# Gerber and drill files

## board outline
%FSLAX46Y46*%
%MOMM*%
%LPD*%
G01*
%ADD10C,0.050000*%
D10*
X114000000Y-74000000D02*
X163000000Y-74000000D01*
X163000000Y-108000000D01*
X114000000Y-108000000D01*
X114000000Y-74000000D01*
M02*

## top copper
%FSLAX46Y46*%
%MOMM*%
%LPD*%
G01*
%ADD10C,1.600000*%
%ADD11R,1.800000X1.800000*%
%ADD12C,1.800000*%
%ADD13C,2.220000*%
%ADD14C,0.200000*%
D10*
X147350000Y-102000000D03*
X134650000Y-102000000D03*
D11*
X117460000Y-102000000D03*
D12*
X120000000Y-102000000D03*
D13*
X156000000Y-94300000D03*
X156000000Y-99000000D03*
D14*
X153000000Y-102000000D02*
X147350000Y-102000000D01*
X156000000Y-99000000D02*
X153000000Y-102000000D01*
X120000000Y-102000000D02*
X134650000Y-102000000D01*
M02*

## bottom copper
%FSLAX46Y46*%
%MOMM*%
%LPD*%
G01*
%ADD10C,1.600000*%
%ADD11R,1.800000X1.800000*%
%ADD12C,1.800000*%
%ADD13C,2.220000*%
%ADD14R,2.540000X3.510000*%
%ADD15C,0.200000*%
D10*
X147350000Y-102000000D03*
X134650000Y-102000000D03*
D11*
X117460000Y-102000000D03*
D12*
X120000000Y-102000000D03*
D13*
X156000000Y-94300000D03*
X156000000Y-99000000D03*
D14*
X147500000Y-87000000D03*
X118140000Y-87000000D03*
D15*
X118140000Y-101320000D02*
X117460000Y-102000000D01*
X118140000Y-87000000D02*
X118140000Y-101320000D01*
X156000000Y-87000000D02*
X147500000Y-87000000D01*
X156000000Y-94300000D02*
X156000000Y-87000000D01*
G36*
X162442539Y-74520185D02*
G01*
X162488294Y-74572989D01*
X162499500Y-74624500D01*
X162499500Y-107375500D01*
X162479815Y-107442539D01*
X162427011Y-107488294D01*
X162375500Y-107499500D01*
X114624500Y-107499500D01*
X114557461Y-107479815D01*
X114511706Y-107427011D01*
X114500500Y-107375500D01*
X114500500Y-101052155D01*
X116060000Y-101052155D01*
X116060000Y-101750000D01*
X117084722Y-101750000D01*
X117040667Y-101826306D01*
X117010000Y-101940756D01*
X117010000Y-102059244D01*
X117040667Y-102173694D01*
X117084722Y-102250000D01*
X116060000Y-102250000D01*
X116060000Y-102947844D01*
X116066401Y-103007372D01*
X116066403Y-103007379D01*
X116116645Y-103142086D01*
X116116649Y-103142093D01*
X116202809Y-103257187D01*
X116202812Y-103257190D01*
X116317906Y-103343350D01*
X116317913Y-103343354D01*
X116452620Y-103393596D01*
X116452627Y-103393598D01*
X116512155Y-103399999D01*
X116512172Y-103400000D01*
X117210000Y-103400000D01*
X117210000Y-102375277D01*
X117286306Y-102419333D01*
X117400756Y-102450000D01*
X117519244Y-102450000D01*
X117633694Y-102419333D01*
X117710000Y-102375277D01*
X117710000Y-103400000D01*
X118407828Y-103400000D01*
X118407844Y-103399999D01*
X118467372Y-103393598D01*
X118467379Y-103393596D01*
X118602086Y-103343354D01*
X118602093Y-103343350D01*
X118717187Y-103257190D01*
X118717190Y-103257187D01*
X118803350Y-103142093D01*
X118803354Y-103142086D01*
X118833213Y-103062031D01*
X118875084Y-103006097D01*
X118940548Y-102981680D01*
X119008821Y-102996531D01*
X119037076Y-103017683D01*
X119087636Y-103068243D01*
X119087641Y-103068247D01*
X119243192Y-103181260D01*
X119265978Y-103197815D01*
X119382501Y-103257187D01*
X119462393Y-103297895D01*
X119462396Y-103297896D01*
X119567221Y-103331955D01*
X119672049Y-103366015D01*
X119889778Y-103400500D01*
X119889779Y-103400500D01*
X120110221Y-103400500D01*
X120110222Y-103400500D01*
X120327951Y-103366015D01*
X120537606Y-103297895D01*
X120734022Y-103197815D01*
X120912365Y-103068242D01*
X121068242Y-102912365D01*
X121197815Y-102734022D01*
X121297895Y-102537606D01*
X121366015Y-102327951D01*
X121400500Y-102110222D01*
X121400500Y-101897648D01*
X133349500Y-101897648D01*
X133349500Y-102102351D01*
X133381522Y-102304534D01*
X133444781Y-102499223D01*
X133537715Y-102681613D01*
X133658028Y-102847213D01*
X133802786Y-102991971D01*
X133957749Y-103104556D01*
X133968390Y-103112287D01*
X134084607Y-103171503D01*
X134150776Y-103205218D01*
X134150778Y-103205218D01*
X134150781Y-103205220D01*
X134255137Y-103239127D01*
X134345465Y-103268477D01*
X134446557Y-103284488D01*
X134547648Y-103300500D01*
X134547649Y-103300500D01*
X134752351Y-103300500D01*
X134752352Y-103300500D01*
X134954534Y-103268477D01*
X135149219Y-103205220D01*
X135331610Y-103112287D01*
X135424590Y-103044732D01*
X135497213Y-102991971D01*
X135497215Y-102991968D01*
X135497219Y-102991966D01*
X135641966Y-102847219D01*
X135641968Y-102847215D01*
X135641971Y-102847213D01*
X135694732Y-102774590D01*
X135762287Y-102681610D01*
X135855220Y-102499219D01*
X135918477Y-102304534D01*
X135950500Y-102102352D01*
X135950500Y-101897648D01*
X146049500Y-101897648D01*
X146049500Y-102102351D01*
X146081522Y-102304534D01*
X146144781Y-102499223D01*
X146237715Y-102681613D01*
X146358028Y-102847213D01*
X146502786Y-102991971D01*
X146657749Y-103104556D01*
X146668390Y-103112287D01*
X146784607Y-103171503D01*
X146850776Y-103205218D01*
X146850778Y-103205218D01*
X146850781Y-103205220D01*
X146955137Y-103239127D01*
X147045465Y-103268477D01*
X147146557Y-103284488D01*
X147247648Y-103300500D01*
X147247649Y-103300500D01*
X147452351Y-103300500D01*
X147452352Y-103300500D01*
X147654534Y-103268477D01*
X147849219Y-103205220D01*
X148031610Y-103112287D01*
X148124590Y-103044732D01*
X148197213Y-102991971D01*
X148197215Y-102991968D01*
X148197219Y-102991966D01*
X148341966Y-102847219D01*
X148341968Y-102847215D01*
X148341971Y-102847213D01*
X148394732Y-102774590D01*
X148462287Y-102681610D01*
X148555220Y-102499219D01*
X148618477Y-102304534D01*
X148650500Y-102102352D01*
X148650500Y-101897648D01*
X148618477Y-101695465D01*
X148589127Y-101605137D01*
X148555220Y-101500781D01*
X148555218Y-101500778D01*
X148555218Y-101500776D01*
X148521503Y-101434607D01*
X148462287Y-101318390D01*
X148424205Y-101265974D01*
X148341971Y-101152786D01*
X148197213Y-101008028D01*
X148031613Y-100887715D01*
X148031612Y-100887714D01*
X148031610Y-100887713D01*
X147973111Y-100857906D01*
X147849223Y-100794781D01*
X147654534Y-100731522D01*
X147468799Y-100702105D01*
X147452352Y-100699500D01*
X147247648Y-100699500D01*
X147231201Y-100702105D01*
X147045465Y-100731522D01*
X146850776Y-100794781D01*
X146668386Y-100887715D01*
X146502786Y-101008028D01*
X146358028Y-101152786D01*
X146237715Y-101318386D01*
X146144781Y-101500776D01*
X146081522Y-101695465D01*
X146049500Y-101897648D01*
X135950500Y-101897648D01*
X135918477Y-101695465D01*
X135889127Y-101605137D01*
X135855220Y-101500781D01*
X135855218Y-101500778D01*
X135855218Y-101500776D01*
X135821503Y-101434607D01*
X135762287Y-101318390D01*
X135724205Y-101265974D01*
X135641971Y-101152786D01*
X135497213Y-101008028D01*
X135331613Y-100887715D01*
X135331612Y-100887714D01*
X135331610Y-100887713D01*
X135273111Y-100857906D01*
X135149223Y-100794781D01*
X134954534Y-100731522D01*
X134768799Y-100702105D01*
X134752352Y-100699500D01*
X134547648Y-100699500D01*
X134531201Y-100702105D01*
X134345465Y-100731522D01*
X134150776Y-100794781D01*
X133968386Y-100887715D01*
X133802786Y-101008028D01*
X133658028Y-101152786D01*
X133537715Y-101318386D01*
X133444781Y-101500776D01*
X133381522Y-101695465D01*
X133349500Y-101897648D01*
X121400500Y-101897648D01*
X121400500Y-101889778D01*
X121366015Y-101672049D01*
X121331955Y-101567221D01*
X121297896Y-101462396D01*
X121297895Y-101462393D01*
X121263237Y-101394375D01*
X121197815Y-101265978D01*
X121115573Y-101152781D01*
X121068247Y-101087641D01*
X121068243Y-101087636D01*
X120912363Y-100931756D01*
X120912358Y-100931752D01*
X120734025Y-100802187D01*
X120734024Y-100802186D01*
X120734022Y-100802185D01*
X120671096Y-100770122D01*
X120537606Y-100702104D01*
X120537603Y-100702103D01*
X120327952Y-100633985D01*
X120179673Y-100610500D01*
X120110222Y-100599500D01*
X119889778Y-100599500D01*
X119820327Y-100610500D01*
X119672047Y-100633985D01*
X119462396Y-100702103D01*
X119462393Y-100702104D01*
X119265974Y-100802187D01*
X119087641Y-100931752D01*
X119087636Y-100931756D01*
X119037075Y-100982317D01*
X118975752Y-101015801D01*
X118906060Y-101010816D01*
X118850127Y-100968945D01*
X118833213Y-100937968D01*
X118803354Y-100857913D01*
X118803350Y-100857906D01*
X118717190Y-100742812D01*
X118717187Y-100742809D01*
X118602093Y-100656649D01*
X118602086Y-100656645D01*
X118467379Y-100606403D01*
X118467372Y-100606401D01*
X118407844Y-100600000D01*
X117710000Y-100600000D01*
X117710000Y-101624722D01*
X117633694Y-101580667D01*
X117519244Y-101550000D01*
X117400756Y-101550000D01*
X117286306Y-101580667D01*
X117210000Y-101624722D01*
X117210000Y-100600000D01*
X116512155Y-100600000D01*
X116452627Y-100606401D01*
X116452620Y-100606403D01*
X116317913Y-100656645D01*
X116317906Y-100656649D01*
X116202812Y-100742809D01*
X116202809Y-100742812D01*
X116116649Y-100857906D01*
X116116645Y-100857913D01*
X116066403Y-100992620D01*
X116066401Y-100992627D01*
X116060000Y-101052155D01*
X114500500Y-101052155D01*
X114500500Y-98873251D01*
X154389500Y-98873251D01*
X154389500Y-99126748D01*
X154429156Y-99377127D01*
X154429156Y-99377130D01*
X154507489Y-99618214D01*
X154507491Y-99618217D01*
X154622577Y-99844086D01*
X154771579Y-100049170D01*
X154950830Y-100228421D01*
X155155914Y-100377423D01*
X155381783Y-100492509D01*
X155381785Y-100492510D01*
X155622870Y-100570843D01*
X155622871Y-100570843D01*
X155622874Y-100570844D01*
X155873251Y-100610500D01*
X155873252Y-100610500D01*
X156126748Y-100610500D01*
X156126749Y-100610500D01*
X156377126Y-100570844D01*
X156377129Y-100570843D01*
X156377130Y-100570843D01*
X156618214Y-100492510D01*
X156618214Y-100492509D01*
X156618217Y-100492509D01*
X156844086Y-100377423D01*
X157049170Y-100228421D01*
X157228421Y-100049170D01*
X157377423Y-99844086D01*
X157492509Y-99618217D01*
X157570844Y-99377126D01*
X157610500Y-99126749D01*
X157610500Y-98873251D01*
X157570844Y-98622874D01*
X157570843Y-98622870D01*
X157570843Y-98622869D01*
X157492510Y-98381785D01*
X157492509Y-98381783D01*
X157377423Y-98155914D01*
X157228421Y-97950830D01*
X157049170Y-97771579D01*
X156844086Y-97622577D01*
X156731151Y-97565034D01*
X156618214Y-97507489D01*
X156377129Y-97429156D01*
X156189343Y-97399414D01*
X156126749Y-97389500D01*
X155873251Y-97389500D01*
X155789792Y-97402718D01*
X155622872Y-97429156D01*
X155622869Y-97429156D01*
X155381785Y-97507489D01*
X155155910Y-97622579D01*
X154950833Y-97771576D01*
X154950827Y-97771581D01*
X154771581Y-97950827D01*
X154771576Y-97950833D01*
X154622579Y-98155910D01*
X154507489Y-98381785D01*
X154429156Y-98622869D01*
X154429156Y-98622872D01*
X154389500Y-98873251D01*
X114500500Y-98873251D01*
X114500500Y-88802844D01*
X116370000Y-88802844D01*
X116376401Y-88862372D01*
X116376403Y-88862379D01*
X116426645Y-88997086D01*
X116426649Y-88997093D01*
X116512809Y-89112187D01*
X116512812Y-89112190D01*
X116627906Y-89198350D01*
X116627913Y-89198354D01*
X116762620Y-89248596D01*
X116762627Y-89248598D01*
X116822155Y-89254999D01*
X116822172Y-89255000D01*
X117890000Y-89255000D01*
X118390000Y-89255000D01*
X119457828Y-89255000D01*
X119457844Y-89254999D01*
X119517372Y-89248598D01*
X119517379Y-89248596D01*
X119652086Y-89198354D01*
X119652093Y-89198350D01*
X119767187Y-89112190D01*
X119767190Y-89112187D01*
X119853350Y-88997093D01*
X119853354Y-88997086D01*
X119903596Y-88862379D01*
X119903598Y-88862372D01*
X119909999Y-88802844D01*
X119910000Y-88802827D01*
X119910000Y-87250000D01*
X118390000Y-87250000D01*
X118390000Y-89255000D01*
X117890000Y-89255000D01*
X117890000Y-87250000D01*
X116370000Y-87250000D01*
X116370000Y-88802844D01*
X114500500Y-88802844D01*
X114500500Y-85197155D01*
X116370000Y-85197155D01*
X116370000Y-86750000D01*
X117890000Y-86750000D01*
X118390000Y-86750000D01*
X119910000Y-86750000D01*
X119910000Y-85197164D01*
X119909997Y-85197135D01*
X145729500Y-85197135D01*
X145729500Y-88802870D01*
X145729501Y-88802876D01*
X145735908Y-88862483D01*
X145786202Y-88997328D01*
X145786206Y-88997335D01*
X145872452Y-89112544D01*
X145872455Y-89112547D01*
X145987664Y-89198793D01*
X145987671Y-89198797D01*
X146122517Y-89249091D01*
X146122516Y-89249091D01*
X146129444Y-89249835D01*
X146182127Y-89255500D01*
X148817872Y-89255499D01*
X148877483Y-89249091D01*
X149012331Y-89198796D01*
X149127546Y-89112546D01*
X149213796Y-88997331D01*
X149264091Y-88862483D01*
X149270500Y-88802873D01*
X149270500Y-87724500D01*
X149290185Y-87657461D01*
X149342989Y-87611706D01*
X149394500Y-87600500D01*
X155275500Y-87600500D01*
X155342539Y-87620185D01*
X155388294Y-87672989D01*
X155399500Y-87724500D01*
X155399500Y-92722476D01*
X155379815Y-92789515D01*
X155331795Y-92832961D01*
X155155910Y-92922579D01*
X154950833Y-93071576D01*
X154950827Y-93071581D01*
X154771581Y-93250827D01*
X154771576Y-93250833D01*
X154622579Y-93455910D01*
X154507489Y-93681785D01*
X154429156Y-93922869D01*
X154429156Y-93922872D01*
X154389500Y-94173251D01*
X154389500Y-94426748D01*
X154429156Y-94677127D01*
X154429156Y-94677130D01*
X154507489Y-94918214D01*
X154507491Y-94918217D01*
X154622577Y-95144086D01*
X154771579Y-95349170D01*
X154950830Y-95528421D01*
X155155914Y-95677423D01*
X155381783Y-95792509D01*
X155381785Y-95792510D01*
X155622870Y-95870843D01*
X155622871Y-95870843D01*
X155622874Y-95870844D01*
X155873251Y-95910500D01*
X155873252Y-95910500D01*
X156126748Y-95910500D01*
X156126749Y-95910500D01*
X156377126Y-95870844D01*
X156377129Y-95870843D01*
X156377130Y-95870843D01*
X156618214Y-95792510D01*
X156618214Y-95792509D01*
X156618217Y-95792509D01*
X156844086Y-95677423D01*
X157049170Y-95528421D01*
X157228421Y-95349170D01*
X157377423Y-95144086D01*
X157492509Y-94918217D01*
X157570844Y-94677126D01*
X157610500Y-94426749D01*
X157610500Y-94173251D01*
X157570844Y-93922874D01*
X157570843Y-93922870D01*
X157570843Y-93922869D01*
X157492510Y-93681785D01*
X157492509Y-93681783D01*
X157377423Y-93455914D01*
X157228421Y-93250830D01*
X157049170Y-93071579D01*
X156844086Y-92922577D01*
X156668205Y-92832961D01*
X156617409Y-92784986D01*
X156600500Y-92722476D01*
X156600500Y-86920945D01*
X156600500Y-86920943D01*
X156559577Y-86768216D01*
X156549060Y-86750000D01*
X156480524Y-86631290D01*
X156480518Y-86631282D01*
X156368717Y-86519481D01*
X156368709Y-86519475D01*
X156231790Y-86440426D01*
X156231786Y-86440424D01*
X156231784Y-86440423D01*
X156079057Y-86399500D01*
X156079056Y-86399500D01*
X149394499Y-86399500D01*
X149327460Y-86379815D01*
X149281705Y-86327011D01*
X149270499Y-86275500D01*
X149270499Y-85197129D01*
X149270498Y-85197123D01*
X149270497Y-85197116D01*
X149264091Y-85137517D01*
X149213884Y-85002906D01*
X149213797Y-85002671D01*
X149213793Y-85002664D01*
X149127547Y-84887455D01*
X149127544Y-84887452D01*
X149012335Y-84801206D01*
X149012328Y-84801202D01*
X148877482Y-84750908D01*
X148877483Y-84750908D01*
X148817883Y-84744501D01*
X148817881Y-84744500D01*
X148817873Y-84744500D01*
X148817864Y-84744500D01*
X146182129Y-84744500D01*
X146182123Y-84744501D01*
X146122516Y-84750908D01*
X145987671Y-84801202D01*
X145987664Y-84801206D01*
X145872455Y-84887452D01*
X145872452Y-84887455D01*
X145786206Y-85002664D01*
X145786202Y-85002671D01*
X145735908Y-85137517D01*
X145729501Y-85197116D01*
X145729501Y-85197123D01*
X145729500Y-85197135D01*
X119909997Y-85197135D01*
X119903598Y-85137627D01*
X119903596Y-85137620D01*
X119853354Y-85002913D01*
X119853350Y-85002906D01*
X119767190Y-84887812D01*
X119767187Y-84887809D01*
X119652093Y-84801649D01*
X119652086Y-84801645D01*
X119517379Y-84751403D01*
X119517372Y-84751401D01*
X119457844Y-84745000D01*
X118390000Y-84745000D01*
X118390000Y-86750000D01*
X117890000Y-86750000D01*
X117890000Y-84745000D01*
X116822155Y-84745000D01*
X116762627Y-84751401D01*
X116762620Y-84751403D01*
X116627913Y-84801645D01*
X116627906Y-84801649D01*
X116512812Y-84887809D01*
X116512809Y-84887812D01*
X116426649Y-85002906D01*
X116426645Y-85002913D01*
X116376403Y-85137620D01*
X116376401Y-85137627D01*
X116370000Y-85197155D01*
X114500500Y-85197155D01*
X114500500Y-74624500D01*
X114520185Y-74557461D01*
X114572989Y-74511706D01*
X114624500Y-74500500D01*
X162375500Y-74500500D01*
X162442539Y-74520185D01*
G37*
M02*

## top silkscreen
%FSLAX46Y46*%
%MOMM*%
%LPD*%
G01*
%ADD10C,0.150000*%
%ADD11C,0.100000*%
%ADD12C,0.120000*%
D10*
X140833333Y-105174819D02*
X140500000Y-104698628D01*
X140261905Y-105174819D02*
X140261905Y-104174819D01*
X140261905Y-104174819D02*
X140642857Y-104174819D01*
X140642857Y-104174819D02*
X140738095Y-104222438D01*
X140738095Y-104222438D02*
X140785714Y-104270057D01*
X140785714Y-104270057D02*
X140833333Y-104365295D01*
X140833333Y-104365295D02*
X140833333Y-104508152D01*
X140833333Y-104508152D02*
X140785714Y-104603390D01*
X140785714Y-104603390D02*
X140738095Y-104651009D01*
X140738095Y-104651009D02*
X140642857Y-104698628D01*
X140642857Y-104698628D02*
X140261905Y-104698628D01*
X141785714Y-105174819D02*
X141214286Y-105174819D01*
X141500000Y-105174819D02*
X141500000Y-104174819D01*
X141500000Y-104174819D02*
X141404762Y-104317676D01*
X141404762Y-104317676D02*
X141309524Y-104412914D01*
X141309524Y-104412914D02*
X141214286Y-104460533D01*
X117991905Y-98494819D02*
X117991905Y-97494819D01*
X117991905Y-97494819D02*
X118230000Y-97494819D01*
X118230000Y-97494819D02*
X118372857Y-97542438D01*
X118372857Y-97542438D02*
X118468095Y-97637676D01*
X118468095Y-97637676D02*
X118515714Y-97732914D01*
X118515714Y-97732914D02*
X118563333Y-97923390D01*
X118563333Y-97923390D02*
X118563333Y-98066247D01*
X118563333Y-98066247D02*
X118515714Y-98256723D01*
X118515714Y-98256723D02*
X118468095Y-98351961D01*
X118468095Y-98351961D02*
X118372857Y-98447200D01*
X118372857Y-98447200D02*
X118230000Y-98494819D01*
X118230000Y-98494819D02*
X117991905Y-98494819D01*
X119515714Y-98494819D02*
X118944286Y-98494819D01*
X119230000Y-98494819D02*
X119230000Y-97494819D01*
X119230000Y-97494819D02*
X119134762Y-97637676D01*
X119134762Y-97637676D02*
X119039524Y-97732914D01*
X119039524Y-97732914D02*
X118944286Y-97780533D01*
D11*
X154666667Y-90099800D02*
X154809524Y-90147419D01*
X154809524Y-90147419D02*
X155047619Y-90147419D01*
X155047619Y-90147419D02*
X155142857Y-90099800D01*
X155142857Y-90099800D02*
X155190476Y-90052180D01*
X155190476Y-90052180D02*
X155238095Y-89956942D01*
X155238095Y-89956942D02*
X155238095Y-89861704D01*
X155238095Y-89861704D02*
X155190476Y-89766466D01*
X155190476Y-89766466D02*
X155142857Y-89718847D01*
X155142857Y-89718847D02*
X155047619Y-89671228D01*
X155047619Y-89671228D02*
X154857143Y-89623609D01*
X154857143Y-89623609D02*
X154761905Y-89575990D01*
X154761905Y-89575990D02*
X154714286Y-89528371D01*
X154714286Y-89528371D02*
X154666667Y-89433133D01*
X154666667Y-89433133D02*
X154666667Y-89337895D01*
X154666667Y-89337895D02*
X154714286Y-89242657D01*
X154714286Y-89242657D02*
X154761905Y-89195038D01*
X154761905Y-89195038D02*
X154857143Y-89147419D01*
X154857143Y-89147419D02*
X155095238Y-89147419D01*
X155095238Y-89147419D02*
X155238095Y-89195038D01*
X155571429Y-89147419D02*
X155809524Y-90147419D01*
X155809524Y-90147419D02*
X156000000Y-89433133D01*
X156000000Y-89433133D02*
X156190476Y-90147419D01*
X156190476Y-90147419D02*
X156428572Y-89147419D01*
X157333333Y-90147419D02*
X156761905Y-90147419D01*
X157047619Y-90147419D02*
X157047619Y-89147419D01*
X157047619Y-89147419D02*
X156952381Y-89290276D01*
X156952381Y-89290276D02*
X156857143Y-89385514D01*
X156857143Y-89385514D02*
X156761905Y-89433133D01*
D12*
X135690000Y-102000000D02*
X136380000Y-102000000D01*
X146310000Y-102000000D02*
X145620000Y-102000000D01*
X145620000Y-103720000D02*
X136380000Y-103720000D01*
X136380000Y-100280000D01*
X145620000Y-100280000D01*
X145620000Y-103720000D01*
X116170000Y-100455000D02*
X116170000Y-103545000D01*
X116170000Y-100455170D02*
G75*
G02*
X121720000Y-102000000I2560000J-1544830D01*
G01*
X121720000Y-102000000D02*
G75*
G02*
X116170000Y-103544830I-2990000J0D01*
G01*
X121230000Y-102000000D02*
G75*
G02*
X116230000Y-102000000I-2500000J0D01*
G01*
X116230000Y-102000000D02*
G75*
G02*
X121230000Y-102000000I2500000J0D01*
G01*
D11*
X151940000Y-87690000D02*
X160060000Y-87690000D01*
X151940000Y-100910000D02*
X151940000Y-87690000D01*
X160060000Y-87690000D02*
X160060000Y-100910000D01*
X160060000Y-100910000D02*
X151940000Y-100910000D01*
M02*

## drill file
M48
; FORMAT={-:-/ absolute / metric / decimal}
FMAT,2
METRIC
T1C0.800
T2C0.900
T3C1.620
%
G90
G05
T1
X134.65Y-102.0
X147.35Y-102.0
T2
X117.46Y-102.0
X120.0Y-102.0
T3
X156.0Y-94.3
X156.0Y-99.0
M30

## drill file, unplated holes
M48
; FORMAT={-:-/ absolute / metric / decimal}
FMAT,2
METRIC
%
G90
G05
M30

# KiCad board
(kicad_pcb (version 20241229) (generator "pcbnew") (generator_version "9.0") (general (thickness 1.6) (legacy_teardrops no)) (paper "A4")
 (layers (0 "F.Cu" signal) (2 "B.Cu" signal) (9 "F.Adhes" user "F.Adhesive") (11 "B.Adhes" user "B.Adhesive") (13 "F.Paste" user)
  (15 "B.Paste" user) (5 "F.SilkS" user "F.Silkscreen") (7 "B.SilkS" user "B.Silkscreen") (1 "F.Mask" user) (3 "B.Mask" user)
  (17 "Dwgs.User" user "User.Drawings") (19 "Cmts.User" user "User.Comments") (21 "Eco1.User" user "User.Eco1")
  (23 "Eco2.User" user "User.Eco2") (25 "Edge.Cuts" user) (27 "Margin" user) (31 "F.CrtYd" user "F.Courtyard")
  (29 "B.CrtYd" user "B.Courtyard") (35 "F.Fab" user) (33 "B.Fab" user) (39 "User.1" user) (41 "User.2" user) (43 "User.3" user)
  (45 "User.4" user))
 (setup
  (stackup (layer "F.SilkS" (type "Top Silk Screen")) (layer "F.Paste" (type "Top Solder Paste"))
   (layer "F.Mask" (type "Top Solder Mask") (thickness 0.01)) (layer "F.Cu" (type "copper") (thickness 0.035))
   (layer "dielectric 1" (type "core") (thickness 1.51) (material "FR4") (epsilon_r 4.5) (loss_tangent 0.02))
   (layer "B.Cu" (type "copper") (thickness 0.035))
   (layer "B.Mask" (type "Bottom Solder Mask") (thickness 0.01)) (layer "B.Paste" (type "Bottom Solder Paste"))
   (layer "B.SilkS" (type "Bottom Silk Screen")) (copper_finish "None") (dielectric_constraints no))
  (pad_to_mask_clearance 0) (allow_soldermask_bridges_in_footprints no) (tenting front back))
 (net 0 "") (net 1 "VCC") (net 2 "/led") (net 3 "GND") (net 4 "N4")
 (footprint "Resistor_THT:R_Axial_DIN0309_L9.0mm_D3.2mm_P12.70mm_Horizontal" (layer "F.Cu") (at 147.35 102 180)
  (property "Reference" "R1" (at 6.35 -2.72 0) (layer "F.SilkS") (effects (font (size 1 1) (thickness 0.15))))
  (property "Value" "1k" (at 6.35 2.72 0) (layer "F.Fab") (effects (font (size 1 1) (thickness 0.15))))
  (fp_line (start 11.66 0) (end 10.97 0) (stroke (width 0.12) (type solid)) (layer "F.SilkS"))
  (fp_line (start 1.04 0) (end 1.73 0) (stroke (width 0.12) (type solid)) (layer "F.SilkS"))
  (fp_rect (start 1.73 -1.72) (end 10.97 1.72) (stroke (width 0.12) (type solid)) (fill no) (layer "F.SilkS"))
  (pad "1" thru_hole circle (at 0 0 180) (size 1.6 1.6) (drill 0.8) (layers "*.Cu" "*.Mask") (remove_unused_layers no) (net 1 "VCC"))
  (pad "2" thru_hole circle (at 12.7 0 180) (size 1.6 1.6) (drill 0.8) (layers "*.Cu" "*.Mask") (remove_unused_layers no) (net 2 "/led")))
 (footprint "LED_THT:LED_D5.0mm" (layer "F.Cu") (at 117.46 102)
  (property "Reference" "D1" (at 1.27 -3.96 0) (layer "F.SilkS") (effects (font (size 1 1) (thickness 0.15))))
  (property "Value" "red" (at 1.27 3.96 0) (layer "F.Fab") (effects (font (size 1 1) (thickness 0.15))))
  (fp_line (start -1.29 -1.545) (end -1.29 1.545) (stroke (width 0.12) (type solid)) (layer "F.SilkS"))
  (fp_arc (start -1.29 -1.54483) (mid 2.071779 -2.880495) (end 4.26 0) (stroke (width 0.12) (type solid)) (layer "F.SilkS"))
  (fp_arc (start 4.26 0) (mid 2.071779 2.880495) (end -1.29 1.54483) (stroke (width 0.12) (type solid)) (layer "F.SilkS"))
  (fp_circle (center 1.27 0) (end 3.77 0) (stroke (width 0.12) (type solid)) (fill no) (layer "F.SilkS"))
  (pad "1" thru_hole rect (at 0 0) (size 1.8 1.8) (drill 0.9) (layers "*.Cu" "*.Mask") (remove_unused_layers no) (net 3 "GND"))
  (pad "2" thru_hole circle (at 2.54 0) (size 1.8 1.8) (drill 0.9) (layers "*.Cu" "*.Mask") (remove_unused_layers no) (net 2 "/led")))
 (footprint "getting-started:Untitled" (layer "F.Cu") (at 156 89.6)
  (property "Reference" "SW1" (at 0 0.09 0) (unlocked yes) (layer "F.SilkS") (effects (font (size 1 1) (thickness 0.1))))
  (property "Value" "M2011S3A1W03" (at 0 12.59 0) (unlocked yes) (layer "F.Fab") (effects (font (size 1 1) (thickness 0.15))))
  (fp_line (start -4.06 -1.91) (end 4.06 -1.91) (stroke (width 0.1) (type default)) (layer "F.SilkS"))
  (fp_line (start -4.06 11.31) (end -4.06 -1.91) (stroke (width 0.1) (type default)) (layer "F.SilkS"))
  (fp_line (start 4.06 -1.91) (end 4.06 11.31) (stroke (width 0.1) (type default)) (layer "F.SilkS"))
  (fp_line (start 4.06 11.31) (end -4.06 11.31) (stroke (width 0.1) (type default)) (layer "F.SilkS"))
  (pad "2" thru_hole circle (at 0 4.7) (size 2.22 2.22) (drill 1.62) (layers "*.Cu" "*.Mask") (remove_unused_layers no) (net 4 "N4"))
  (pad "3" thru_hole circle (at 0 9.4) (size 2.22 2.22) (drill 1.62) (layers "*.Cu" "*.Mask") (remove_unused_layers no) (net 1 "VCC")))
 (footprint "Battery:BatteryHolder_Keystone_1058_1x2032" (layer "B.Cu") (at 132.82 87 180)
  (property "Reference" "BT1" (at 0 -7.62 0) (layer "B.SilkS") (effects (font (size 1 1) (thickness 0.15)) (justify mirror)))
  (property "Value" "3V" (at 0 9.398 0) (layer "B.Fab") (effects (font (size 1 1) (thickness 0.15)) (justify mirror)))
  (pad "1" smd rect (at -14.68 0 180) (size 2.54 3.51) (layers "B.Cu" "B.Mask" "B.Paste") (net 4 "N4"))
  (pad "2" smd rect (at 14.68 0 180) (size 2.54 3.51) (layers "B.Cu" "B.Mask" "B.Paste") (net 3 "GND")))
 (gr_rect (start 114 74) (end 163 108) (stroke (width 0.05) (type default)) (fill no) (layer "Edge.Cuts"))
 (segment (start 153 102) (end 147.35 102) (width 0.2) (layer "F.Cu") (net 1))
 (segment (start 156 99) (end 153 102) (width 0.2) (layer "F.Cu") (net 1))
 (segment (start 118.14 101.32) (end 117.46 102) (width 0.2) (layer "B.Cu") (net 3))
 (segment (start 118.14 87) (end 118.14 101.32) (width 0.2) (layer "B.Cu") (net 3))
 (segment (start 120 102) (end 134.65 102) (width 0.2) (layer "F.Cu") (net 2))
 (segment (start 156 87) (end 147.5 87) (width 0.2) (layer "B.Cu") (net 4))
 (segment (start 156 94.3) (end 156 87) (width 0.2) (layer "B.Cu") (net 4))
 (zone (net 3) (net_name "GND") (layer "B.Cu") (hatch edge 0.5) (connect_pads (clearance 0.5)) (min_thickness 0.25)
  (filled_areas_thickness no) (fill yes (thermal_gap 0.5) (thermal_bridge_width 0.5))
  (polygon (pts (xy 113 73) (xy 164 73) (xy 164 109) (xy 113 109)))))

